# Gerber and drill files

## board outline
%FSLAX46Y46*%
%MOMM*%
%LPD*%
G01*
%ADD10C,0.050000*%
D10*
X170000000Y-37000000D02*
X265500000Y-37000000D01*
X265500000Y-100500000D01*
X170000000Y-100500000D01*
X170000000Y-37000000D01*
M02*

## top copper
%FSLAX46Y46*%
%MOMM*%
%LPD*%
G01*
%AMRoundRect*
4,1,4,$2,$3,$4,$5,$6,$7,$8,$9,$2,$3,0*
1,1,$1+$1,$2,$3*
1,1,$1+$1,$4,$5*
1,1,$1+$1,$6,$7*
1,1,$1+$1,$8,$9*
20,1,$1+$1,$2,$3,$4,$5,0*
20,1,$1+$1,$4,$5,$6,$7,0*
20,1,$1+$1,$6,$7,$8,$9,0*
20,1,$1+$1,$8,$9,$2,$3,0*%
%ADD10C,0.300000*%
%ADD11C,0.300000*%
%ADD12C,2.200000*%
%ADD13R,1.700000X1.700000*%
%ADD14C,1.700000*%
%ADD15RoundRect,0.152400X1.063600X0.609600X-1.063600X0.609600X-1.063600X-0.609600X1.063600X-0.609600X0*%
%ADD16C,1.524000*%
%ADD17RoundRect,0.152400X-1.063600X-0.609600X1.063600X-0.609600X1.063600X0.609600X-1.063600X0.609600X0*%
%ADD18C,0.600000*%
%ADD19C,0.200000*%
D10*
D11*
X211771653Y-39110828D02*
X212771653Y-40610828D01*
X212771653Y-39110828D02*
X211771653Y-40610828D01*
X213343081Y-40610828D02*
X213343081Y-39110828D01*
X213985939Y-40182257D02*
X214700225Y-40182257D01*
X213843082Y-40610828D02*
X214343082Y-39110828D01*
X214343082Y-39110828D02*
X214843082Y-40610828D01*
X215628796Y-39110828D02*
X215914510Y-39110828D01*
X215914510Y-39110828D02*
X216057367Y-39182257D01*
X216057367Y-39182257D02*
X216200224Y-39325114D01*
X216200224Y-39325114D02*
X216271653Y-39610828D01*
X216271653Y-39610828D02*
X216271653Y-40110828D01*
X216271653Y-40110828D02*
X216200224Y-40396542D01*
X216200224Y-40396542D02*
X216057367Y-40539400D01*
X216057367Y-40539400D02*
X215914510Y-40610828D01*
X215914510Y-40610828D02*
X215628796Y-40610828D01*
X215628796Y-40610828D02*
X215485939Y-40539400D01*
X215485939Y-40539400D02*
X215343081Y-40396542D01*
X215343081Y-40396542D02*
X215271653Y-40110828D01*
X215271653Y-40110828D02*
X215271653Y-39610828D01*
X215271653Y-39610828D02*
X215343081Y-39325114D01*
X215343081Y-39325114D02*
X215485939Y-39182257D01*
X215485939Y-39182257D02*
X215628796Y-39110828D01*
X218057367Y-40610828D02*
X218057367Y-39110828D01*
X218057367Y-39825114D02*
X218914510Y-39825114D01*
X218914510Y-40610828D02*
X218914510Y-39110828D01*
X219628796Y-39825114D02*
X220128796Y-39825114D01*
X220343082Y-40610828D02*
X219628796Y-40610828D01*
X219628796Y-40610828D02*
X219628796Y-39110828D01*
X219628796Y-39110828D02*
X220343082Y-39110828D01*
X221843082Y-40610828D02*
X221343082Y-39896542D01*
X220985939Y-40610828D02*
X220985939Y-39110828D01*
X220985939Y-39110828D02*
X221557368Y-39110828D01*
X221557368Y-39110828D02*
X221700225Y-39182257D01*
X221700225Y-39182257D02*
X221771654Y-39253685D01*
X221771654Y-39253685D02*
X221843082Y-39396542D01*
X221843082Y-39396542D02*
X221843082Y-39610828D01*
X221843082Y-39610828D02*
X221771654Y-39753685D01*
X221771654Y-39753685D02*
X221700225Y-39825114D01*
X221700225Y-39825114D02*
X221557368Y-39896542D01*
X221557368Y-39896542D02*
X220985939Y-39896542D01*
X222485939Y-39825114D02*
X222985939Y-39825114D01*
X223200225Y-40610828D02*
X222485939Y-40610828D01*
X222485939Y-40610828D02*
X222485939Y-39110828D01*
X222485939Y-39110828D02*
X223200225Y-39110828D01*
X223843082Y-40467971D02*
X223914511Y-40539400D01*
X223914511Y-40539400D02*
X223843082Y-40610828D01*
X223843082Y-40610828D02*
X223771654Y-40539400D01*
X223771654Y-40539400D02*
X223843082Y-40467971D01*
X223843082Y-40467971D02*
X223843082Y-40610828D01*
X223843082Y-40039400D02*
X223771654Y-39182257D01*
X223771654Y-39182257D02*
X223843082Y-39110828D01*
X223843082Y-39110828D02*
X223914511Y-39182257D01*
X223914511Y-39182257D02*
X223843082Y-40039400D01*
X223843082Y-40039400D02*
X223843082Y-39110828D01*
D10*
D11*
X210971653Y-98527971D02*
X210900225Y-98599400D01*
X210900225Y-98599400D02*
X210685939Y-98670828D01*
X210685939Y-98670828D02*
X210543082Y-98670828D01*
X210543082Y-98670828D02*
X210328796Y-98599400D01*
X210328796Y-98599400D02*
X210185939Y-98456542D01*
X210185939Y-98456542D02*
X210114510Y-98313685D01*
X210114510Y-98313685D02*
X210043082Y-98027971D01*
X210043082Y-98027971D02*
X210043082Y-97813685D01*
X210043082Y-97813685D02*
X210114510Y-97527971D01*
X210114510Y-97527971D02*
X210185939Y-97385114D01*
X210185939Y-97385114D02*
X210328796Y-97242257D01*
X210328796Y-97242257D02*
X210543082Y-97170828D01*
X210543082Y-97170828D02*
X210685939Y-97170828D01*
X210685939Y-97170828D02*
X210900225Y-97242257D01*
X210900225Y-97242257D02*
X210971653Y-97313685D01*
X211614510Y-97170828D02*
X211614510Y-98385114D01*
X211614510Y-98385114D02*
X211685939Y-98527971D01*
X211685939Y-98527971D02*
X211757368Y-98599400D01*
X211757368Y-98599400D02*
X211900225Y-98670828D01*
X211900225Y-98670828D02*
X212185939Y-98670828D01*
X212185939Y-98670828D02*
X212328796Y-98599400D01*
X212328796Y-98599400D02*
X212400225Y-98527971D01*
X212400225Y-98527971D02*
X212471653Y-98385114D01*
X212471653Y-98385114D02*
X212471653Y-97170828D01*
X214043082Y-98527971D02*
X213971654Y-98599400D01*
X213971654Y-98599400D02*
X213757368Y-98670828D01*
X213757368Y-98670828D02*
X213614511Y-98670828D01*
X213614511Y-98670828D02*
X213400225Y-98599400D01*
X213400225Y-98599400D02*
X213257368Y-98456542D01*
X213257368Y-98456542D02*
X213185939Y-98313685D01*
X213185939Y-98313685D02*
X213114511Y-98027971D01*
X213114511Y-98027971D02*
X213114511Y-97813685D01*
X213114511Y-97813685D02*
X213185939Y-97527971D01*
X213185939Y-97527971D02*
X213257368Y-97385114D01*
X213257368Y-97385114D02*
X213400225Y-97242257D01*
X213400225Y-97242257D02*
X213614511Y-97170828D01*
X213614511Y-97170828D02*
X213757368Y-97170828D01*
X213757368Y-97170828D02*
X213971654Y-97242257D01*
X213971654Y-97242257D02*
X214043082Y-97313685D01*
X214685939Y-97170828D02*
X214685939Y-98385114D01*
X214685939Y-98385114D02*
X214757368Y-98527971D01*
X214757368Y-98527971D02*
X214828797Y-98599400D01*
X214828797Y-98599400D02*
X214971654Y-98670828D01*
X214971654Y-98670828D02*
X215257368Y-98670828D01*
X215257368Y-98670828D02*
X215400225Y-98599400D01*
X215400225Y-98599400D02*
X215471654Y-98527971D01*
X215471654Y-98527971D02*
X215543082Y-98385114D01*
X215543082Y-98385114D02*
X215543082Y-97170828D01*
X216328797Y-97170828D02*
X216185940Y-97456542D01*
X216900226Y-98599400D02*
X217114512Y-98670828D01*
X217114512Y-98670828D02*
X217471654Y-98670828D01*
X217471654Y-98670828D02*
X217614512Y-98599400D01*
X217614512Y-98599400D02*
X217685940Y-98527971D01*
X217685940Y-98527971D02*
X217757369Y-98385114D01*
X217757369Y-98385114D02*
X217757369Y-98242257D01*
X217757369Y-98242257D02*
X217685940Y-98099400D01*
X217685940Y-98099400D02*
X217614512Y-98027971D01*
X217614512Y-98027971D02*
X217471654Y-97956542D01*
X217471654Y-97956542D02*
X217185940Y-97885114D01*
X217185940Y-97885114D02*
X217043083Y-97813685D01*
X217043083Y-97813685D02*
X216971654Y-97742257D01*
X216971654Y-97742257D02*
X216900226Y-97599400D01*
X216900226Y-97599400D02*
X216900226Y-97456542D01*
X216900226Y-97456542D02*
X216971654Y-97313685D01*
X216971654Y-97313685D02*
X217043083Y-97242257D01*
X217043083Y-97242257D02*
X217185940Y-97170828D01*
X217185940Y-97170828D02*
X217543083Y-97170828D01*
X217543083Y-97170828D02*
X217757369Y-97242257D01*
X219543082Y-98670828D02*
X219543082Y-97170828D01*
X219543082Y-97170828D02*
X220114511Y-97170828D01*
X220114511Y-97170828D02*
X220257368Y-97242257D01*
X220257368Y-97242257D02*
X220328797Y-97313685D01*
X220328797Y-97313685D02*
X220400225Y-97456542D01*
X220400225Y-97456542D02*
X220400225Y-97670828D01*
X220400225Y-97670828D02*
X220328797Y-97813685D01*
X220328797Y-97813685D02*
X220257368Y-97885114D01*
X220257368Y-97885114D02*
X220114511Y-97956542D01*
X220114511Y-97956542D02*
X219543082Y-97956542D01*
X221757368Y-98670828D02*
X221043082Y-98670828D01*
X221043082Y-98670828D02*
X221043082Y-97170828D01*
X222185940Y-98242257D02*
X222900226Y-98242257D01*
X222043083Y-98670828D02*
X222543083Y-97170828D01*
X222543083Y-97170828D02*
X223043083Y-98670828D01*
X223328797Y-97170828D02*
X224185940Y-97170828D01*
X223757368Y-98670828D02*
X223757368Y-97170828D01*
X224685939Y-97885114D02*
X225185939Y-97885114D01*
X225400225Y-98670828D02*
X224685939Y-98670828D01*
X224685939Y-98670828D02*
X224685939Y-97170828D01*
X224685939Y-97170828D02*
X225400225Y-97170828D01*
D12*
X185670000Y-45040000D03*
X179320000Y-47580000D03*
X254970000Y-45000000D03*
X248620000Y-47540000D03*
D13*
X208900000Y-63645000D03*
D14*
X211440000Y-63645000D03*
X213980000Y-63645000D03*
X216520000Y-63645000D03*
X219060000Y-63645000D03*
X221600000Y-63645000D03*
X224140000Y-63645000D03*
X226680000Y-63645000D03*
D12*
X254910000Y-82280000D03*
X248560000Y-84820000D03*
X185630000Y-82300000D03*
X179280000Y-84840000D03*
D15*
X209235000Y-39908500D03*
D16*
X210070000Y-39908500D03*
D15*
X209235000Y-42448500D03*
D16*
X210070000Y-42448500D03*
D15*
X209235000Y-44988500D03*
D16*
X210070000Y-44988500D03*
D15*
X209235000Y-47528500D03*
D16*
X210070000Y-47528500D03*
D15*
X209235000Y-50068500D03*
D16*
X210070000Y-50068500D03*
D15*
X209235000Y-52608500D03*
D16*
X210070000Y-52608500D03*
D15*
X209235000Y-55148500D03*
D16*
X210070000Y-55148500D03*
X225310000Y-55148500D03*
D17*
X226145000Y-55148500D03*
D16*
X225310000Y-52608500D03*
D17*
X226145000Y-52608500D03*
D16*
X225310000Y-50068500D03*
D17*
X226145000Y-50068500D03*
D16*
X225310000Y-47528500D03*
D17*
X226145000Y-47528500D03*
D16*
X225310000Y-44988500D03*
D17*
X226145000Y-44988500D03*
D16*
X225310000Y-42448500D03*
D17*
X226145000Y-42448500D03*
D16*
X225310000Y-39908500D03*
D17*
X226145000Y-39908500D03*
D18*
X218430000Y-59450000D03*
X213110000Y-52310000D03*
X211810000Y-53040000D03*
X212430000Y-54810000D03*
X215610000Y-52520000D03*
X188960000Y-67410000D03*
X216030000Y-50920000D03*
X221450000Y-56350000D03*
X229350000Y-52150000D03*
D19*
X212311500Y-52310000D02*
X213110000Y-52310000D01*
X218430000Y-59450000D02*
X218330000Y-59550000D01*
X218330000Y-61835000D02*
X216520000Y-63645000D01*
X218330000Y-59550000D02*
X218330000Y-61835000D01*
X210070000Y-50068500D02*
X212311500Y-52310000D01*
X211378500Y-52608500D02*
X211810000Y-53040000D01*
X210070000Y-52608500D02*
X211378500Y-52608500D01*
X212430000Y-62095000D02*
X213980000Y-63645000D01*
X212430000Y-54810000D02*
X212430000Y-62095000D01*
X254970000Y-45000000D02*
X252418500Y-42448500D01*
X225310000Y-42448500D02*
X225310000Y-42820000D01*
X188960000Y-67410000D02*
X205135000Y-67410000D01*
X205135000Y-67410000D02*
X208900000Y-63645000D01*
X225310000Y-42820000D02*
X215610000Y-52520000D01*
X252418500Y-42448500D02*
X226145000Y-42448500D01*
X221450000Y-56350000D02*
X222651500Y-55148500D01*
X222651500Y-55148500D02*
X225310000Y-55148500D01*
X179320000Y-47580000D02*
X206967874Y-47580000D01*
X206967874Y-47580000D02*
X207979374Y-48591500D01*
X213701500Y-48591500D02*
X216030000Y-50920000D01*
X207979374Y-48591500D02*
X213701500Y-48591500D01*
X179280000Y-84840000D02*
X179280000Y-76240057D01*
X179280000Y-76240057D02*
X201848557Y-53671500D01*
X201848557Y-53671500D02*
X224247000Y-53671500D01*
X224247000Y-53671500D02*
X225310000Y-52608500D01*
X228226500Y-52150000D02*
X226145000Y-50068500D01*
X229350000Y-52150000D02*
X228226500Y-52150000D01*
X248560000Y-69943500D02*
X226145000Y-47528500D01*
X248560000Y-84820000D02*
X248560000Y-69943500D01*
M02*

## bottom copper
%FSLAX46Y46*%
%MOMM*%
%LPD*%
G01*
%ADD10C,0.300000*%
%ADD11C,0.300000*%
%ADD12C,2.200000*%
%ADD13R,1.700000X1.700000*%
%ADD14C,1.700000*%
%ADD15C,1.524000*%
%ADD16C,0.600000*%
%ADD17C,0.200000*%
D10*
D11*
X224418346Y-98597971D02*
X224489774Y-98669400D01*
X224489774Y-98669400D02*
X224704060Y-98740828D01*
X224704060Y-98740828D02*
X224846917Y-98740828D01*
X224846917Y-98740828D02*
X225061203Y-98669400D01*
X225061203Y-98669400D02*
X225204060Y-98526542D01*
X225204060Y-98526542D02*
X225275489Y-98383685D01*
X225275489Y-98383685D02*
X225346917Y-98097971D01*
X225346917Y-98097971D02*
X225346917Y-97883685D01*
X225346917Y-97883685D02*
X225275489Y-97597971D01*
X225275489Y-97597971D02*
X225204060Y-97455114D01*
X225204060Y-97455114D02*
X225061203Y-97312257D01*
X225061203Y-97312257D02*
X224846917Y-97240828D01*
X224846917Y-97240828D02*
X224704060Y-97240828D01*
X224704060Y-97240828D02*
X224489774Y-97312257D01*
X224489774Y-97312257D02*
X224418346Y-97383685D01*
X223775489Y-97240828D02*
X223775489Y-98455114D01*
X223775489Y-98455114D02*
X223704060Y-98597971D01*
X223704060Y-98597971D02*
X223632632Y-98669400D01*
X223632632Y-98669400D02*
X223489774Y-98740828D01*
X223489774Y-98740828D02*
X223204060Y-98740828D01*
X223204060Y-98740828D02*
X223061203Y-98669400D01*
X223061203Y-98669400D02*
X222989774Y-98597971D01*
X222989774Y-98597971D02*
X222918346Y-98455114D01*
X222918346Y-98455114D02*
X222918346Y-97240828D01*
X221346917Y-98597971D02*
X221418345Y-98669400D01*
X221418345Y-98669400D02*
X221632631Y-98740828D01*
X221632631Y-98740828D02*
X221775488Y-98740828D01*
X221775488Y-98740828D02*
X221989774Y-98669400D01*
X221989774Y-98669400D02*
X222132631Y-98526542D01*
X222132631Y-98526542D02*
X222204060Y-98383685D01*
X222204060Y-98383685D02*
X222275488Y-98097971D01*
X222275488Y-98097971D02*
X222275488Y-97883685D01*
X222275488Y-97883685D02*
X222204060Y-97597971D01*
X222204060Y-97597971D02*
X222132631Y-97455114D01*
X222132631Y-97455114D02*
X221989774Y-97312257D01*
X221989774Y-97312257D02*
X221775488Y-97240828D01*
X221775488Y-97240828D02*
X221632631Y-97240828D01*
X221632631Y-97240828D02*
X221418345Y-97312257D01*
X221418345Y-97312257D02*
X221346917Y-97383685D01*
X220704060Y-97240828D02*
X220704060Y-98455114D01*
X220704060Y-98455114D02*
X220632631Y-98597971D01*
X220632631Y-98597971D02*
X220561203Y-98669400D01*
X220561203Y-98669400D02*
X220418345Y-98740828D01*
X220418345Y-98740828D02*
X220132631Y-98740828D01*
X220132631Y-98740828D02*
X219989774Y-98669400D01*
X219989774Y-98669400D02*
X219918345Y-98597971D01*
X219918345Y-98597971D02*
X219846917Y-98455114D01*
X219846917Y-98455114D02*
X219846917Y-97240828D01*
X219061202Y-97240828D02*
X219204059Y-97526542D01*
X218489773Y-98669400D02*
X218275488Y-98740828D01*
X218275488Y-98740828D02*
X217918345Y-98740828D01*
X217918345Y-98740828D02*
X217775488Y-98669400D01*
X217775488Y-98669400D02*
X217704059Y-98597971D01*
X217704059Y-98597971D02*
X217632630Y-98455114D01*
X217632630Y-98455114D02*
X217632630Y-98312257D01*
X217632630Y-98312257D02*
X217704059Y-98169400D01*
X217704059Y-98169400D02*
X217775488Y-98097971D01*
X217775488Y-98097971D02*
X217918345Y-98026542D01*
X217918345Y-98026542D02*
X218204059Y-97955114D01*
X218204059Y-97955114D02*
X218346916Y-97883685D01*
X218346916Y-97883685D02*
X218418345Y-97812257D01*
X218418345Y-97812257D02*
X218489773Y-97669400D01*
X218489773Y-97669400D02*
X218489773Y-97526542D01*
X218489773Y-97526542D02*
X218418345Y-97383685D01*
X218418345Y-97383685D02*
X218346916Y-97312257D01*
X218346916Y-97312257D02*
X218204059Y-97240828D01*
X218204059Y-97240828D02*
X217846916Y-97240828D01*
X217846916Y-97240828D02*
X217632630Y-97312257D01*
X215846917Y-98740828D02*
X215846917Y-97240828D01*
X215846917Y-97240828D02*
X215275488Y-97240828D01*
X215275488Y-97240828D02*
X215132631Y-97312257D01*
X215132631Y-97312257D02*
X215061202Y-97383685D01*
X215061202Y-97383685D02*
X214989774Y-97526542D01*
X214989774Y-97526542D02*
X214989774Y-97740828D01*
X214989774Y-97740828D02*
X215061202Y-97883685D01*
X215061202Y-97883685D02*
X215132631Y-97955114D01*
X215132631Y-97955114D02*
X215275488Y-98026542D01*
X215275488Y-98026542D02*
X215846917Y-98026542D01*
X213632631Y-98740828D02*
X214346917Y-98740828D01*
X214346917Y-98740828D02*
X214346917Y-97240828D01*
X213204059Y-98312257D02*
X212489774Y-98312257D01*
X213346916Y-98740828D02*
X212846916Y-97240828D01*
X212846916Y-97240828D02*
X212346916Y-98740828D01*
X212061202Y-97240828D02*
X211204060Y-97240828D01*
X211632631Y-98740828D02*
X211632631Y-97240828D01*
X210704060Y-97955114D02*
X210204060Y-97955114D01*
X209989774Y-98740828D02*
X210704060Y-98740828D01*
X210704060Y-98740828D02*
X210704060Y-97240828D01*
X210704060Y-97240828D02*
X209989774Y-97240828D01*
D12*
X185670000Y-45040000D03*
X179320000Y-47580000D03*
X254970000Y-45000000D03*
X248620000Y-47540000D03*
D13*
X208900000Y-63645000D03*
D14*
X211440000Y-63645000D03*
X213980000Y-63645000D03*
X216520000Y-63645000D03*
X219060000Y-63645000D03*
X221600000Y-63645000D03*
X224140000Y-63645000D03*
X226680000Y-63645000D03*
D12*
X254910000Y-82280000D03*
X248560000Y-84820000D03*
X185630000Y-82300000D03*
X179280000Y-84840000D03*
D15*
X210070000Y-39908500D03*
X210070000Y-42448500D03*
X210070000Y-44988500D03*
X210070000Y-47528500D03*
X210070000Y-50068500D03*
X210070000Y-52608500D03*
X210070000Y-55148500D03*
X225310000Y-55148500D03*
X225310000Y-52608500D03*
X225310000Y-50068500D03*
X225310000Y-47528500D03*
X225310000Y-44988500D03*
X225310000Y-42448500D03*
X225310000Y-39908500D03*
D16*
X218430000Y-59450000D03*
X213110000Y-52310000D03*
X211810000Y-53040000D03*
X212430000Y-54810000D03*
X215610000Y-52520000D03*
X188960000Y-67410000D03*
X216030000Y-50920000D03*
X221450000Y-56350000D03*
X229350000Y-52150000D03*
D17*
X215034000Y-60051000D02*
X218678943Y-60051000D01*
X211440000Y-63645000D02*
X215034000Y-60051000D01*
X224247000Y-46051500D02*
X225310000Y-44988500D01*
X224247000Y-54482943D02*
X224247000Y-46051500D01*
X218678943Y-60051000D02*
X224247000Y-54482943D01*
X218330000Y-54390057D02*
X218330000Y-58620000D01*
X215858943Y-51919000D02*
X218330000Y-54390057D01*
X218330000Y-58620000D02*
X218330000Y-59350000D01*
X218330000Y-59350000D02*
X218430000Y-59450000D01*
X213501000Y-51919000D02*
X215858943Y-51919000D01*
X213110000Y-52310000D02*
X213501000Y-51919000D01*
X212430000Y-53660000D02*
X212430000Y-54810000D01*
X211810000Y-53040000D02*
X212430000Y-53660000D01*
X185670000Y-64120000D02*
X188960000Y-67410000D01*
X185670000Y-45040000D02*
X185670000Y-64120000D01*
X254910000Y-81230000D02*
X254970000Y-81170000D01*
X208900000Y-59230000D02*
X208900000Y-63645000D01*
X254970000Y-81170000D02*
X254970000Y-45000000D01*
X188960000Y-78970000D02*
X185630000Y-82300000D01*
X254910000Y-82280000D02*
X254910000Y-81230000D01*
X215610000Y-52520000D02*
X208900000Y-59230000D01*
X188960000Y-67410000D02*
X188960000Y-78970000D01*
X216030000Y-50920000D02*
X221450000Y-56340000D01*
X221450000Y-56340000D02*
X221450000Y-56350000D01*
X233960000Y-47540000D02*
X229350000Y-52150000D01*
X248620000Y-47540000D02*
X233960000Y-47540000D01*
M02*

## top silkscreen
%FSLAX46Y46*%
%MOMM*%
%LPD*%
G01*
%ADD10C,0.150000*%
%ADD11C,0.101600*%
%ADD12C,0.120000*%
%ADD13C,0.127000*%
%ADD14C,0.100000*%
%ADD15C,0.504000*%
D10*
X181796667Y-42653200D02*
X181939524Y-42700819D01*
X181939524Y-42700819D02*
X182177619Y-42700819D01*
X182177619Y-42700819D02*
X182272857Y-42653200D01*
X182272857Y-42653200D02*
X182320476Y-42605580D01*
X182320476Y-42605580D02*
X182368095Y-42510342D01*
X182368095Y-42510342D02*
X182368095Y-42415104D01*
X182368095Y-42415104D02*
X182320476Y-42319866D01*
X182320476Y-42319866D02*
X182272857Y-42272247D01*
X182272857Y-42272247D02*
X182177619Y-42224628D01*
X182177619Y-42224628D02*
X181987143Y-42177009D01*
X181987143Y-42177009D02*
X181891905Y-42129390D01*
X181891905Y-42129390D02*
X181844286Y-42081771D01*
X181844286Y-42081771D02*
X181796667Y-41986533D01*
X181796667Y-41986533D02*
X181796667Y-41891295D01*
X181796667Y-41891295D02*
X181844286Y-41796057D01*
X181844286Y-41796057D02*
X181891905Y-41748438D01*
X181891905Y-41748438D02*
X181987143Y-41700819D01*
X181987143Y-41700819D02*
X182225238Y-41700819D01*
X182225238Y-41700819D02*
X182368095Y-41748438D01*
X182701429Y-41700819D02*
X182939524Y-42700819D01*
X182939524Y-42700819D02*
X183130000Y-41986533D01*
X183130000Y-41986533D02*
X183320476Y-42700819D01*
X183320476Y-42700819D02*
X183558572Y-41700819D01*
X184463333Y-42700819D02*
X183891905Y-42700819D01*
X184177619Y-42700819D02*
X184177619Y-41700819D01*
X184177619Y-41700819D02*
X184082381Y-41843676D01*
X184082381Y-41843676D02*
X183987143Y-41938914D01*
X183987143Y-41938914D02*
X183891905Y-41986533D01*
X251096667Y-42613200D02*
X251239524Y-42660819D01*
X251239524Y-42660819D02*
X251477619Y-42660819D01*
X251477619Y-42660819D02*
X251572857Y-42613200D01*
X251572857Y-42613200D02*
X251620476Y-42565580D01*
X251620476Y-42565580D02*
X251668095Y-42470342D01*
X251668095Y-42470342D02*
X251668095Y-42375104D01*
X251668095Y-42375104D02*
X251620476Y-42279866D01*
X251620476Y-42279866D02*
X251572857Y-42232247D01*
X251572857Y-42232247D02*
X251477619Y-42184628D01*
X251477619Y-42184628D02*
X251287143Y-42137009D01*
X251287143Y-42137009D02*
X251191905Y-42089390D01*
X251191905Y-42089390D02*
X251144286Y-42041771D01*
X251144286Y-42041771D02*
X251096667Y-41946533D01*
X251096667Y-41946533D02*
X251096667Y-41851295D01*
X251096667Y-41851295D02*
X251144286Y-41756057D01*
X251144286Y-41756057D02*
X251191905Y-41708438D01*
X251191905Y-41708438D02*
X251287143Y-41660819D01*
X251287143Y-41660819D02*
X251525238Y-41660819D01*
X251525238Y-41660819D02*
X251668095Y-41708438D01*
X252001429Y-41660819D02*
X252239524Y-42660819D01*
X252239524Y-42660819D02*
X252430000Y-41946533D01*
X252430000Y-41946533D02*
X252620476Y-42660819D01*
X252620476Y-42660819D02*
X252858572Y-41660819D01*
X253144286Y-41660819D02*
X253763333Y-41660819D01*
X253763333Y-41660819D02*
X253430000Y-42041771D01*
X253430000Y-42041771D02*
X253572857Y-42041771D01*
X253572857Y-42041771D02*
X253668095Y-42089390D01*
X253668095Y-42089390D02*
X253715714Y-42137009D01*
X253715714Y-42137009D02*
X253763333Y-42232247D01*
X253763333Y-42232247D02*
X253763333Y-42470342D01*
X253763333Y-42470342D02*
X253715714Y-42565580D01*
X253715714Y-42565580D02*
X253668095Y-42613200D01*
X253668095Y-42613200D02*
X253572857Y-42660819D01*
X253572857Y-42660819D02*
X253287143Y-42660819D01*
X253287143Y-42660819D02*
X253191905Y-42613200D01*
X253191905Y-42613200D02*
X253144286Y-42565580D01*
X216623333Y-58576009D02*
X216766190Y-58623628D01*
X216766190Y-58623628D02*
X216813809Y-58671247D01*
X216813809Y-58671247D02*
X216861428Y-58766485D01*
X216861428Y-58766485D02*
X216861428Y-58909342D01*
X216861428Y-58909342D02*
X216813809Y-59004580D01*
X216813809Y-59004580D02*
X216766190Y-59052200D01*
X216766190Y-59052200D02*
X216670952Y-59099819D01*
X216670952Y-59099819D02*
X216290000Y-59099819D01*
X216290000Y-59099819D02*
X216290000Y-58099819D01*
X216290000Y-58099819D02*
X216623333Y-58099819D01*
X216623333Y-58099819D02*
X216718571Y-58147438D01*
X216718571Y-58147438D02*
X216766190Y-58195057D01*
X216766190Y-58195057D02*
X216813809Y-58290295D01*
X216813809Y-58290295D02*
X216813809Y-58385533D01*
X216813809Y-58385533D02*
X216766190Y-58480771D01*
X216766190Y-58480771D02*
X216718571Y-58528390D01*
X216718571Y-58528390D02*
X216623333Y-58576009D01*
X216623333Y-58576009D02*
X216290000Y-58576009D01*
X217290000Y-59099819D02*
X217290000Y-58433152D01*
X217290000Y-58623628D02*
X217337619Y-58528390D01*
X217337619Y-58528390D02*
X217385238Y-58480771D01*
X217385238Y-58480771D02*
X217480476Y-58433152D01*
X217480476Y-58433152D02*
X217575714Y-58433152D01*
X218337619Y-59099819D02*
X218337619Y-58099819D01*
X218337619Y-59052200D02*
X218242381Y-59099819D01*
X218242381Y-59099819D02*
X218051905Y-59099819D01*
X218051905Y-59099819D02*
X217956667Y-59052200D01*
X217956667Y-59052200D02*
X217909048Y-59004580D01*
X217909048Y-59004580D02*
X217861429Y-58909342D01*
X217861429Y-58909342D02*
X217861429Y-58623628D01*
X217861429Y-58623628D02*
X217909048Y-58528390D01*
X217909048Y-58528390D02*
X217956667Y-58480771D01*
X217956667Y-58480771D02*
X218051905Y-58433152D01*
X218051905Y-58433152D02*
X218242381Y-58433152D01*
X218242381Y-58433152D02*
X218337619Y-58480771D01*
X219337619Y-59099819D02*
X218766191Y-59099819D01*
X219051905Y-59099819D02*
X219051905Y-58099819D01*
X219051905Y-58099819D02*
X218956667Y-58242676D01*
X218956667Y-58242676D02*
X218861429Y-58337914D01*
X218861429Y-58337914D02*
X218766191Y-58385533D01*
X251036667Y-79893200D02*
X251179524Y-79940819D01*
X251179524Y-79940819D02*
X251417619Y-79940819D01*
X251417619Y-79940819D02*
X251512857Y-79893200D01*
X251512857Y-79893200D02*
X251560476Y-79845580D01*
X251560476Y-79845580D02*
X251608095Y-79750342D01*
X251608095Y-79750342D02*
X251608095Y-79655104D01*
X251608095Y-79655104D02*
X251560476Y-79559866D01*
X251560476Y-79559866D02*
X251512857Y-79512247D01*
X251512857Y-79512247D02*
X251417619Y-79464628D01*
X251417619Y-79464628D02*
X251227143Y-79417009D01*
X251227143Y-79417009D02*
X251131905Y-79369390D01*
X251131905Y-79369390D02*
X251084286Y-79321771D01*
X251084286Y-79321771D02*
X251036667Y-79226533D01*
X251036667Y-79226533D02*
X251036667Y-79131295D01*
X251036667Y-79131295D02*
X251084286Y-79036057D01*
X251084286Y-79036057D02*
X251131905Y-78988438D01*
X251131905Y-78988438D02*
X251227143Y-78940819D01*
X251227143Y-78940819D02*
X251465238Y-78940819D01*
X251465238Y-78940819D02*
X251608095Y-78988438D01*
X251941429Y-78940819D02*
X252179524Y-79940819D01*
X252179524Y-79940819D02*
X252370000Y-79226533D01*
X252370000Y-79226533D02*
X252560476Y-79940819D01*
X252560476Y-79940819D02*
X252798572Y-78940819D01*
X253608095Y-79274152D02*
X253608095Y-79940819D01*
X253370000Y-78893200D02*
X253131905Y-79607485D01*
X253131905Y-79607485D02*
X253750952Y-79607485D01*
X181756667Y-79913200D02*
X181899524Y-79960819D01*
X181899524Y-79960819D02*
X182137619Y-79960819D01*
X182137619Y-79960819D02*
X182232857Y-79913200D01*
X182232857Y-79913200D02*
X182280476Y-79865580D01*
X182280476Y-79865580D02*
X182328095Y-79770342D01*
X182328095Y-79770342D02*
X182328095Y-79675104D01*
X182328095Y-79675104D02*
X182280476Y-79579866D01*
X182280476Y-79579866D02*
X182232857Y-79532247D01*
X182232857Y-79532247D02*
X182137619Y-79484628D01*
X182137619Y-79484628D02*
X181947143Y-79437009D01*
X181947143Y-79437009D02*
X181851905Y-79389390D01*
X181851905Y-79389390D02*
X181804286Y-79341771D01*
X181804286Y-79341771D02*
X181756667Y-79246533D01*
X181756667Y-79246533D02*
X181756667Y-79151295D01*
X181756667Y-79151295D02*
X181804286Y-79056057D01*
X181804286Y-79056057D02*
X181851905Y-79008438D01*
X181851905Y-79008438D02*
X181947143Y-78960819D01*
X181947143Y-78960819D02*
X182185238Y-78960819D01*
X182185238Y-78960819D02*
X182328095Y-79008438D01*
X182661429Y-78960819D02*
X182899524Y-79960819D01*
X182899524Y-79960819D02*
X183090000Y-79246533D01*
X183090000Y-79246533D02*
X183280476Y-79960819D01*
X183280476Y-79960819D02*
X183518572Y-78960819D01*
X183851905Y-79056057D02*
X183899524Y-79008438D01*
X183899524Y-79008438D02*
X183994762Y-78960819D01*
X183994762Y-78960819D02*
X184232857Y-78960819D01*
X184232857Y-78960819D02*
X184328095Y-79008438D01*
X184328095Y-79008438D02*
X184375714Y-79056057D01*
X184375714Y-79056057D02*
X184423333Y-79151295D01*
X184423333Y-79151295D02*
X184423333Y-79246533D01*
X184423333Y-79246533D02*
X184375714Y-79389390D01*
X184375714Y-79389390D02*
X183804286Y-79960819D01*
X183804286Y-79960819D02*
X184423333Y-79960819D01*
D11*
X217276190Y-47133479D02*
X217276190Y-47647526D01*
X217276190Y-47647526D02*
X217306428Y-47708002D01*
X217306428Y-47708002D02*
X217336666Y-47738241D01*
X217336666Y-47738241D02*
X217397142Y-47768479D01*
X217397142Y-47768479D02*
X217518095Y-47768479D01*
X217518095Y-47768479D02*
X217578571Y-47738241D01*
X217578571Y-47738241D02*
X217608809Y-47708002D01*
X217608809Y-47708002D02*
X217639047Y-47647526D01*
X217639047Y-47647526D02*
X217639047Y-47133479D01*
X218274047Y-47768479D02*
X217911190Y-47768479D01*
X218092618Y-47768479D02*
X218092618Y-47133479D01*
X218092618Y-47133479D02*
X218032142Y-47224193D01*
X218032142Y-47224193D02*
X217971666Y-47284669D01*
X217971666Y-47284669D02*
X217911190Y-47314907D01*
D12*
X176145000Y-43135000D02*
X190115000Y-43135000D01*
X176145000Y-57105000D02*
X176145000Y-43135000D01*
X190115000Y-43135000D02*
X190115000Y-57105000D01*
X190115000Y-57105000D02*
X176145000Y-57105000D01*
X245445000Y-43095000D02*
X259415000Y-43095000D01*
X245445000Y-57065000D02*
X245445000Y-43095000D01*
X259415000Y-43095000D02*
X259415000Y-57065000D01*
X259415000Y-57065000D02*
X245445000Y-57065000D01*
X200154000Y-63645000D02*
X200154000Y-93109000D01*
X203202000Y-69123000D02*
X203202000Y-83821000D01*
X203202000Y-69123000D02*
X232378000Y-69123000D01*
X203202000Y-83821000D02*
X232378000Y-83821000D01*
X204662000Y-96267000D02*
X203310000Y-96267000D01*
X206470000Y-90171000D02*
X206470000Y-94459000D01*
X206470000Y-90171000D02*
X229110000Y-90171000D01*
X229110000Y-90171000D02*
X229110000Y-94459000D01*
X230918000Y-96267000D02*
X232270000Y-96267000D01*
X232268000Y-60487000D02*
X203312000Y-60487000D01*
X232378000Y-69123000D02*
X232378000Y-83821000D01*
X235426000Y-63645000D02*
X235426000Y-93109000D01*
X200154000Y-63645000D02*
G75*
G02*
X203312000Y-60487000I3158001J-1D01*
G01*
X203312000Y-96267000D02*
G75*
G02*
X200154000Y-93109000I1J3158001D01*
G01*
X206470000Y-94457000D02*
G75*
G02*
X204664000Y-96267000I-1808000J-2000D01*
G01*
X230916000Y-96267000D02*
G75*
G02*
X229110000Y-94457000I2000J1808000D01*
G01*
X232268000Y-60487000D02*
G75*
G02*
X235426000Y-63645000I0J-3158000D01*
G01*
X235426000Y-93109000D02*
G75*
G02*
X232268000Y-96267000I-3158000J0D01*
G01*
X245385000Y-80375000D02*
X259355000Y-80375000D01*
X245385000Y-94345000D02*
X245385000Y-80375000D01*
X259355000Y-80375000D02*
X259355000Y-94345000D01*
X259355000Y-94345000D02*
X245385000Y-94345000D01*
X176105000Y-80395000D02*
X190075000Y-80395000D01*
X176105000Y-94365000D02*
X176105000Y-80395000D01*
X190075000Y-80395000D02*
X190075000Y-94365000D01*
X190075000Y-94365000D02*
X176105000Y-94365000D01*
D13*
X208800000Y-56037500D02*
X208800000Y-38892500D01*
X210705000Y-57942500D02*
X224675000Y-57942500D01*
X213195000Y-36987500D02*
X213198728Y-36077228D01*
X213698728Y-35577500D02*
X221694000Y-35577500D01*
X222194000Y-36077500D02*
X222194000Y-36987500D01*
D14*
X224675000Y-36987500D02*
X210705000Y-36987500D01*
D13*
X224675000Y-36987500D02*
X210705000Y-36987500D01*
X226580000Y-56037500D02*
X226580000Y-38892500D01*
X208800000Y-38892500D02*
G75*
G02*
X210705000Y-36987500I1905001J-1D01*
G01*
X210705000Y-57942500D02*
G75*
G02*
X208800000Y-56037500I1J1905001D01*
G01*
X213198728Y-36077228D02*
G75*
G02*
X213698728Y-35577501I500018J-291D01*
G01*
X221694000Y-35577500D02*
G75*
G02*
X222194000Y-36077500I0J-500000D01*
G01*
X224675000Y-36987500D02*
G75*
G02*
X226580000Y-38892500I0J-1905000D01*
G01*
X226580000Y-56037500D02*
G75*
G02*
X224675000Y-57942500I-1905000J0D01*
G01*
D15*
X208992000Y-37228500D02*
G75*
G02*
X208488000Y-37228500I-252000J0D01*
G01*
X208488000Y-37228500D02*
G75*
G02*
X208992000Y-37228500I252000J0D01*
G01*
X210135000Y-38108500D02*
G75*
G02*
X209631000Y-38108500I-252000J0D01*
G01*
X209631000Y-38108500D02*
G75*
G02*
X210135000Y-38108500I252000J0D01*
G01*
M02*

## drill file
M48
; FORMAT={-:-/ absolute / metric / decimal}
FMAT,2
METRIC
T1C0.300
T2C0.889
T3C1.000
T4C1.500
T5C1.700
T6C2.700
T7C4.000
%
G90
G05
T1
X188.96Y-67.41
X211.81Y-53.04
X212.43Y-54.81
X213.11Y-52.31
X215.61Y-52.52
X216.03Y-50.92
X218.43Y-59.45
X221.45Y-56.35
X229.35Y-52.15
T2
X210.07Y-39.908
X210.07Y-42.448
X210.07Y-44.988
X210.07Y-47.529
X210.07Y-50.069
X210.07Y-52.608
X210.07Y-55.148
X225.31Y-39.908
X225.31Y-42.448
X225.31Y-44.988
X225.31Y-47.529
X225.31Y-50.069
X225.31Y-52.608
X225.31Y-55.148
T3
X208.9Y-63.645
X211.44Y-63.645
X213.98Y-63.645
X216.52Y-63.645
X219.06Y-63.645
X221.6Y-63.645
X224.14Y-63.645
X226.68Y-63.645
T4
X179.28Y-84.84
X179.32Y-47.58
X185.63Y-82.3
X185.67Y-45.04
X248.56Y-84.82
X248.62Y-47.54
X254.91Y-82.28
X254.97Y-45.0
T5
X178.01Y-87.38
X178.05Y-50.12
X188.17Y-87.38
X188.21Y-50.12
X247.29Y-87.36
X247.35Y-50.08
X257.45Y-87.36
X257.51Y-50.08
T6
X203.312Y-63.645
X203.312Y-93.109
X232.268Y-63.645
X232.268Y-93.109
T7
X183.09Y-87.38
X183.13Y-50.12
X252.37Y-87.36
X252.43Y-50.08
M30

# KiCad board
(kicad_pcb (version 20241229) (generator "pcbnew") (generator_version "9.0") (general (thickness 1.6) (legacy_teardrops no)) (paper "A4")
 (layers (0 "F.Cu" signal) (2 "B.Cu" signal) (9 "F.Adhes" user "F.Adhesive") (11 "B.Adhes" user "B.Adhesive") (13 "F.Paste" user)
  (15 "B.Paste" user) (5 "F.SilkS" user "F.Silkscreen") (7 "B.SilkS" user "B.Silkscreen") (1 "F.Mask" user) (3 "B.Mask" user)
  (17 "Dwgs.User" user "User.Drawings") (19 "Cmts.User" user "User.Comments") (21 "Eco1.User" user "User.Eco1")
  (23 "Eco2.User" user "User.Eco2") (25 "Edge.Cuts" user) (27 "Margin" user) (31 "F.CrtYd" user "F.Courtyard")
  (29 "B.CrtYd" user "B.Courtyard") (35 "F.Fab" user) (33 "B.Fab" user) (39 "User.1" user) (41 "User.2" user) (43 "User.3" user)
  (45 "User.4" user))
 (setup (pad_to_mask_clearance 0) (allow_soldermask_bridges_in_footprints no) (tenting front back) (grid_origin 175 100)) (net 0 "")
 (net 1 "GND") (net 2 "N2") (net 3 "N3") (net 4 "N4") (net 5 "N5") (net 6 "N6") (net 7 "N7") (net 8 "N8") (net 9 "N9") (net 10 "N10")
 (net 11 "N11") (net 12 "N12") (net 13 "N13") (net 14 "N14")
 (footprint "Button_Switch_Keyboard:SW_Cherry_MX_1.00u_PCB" (layer "F.Cu") (at 185.67 45.04)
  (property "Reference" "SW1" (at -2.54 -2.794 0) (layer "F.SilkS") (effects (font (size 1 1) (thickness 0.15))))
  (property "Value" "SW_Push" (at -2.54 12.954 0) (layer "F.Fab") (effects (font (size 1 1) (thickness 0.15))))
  (fp_line (start -9.525 -1.905) (end 4.445 -1.905) (stroke (width 0.12) (type solid)) (layer "F.SilkS"))
  (fp_line (start -9.525 12.065) (end -9.525 -1.905) (stroke (width 0.12) (type solid)) (layer "F.SilkS"))
  (fp_line (start 4.445 -1.905) (end 4.445 12.065) (stroke (width 0.12) (type solid)) (layer "F.SilkS"))
  (fp_line (start 4.445 12.065) (end -9.525 12.065) (stroke (width 0.12) (type solid)) (layer "F.SilkS"))
  (pad "" np_thru_hole circle (at -7.62 5.08) (size 1.7 1.7) (drill 1.7) (layers "*.Cu" "*.Mask"))
  (pad "" np_thru_hole circle (at -2.54 5.08) (size 4 4) (drill 4) (layers "*.Cu" "*.Mask"))
  (pad "" np_thru_hole circle (at 2.54 5.08) (size 1.7 1.7) (drill 1.7) (layers "*.Cu" "*.Mask"))
  (pad "1" thru_hole circle (at 0 0) (size 2.2 2.2) (drill 1.5) (layers "*.Cu" "*.Mask") (remove_unused_layers no) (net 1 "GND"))
  (pad "2" thru_hole circle (at -6.35 2.54) (size 2.2 2.2) (drill 1.5) (layers "*.Cu" "*.Mask") (remove_unused_layers no) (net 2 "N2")))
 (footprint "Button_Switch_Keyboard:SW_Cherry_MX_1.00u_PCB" (layer "F.Cu") (at 254.97 45)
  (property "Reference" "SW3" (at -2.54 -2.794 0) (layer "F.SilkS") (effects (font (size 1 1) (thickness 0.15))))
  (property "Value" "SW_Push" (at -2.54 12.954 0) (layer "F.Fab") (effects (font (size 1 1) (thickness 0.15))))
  (fp_line (start -9.525 -1.905) (end 4.445 -1.905) (stroke (width 0.12) (type solid)) (layer "F.SilkS"))
  (fp_line (start -9.525 12.065) (end -9.525 -1.905) (stroke (width 0.12) (type solid)) (layer "F.SilkS"))
  (fp_line (start 4.445 -1.905) (end 4.445 12.065) (stroke (width 0.12) (type solid)) (layer "F.SilkS"))
  (fp_line (start 4.445 12.065) (end -9.525 12.065) (stroke (width 0.12) (type solid)) (layer "F.SilkS"))
  (pad "" np_thru_hole circle (at -7.62 5.08) (size 1.7 1.7) (drill 1.7) (layers "*.Cu" "*.Mask"))
  (pad "" np_thru_hole circle (at -2.54 5.08) (size 4 4) (drill 4) (layers "*.Cu" "*.Mask"))
  (pad "" np_thru_hole circle (at 2.54 5.08) (size 1.7 1.7) (drill 1.7) (layers "*.Cu" "*.Mask"))
  (pad "1" thru_hole circle (at 0 0) (size 2.2 2.2) (drill 1.5) (layers "*.Cu" "*.Mask") (remove_unused_layers no) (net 1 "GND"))
  (pad "2" thru_hole circle (at -6.35 2.54) (size 2.2 2.2) (drill 1.5) (layers "*.Cu" "*.Mask") (remove_unused_layers no) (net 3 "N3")))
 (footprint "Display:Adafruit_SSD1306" (layer "F.Cu") (at 208.9 63.645)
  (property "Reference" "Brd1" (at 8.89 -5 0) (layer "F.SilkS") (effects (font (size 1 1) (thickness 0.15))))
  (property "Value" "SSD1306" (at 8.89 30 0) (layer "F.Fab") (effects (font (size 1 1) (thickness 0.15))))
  (fp_line (start -8.746 0) (end -8.746 29.464) (stroke (width 0.12) (type solid)) (layer "F.SilkS"))
  (fp_line (start -5.698 5.478) (end -5.698 20.176) (stroke (width 0.12) (type solid)) (layer "F.SilkS"))
  (fp_line (start -5.698 5.478) (end 23.478 5.478) (stroke (width 0.12) (type solid)) (layer "F.SilkS"))
  (fp_line (start -5.698 20.176) (end 23.478 20.176) (stroke (width 0.12) (type solid)) (layer "F.SilkS"))
  (fp_line (start -4.238 32.622) (end -5.59 32.622) (stroke (width 0.12) (type solid)) (layer "F.SilkS"))
  (fp_line (start -2.43 26.526) (end -2.43 30.814) (stroke (width 0.12) (type solid)) (layer "F.SilkS"))
  (fp_line (start -2.43 26.526) (end 20.21 26.526) (stroke (width 0.12) (type solid)) (layer "F.SilkS"))
  (fp_line (start 20.21 26.526) (end 20.21 30.814) (stroke (width 0.12) (type solid)) (layer "F.SilkS"))
  (fp_line (start 22.018 32.622) (end 23.37 32.622) (stroke (width 0.12) (type solid)) (layer "F.SilkS"))
  (fp_line (start 23.368 -3.158) (end -5.588 -3.158) (stroke (width 0.12) (type solid)) (layer "F.SilkS"))
  (fp_line (start 23.478 5.478) (end 23.478 20.176) (stroke (width 0.12) (type solid)) (layer "F.SilkS"))
  (fp_line (start 26.526 0) (end 26.526 29.464) (stroke (width 0.12) (type solid)) (layer "F.SilkS"))
  (fp_arc (start -8.746 0) (mid -7.821043 -2.233043) (end -5.588 -3.158) (stroke (width 0.12) (type solid)) (layer "F.SilkS"))
  (fp_arc (start -5.588 32.622) (mid -7.821043 31.697043) (end -8.746 29.464) (stroke (width 0.12) (type solid)) (layer "F.SilkS"))
  (fp_arc (start -2.43 30.812) (mid -2.958137 32.091035) (end -4.236 32.622) (stroke (width 0.12) (type solid)) (layer "F.SilkS"))
  (fp_arc (start 22.016 32.622) (mid 20.738137 32.091035) (end 20.21 30.812) (stroke (width 0.12) (type solid)) (layer "F.SilkS"))
  (fp_arc (start 23.368 -3.158) (mid 25.601043 -2.233043) (end 26.526 0) (stroke (width 0.12) (type solid)) (layer "F.SilkS"))
  (fp_arc (start 26.526 29.464) (mid 25.601043 31.697043) (end 23.368 32.622) (stroke (width 0.12) (type solid)) (layer "F.SilkS"))
  (pad "" np_thru_hole circle (at -5.588 0) (size 2.7 2.7) (drill 2.7) (layers "*.Cu" "*.Mask"))
  (pad "" np_thru_hole circle (at -5.588 29.464) (size 2.7 2.7) (drill 2.7) (layers "*.Cu" "*.Mask"))
  (pad "" np_thru_hole circle (at 23.368 0) (size 2.7 2.7) (drill 2.7) (layers "*.Cu" "*.Mask"))
  (pad "" np_thru_hole circle (at 23.368 29.464) (size 2.7 2.7) (drill 2.7) (layers "*.Cu" "*.Mask"))
  (pad "1" thru_hole rect (at 0 0) (size 1.7 1.7) (drill 1) (layers "*.Cu" "*.Mask") (remove_unused_layers no) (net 1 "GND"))
  (pad "2" thru_hole circle (at 2.54 0) (size 1.7 1.7) (drill 1) (layers "*.Cu" "*.Mask") (remove_unused_layers no) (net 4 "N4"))
  (pad "3" thru_hole circle (at 5.08 0) (size 1.7 1.7) (drill 1) (layers "*.Cu" "*.Mask") (remove_unused_layers no) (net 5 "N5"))
  (pad "4" thru_hole circle (at 7.62 0) (size 1.7 1.7) (drill 1) (layers "*.Cu" "*.Mask") (remove_unused_layers no) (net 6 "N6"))
  (pad "5" thru_hole circle (at 10.16 0) (size 1.7 1.7) (drill 1) (layers "*.Cu" "*.Mask") (remove_unused_layers no))
  (pad "6" thru_hole circle (at 12.7 0) (size 1.7 1.7) (drill 1) (layers "*.Cu" "*.Mask") (remove_unused_layers no))
  (pad "7" thru_hole circle (at 15.24 0) (size 1.7 1.7) (drill 1) (layers "*.Cu" "*.Mask") (remove_unused_layers no))
  (pad "8" thru_hole circle (at 17.78 0) (size 1.7 1.7) (drill 1) (layers "*.Cu" "*.Mask") (remove_unused_layers no)))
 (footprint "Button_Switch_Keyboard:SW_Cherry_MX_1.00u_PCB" (layer "F.Cu") (at 254.91 82.28)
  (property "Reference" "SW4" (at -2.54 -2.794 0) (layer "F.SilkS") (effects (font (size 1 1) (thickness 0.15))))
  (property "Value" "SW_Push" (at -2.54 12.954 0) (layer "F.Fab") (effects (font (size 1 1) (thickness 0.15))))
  (fp_line (start -9.525 -1.905) (end 4.445 -1.905) (stroke (width 0.12) (type solid)) (layer "F.SilkS"))
  (fp_line (start -9.525 12.065) (end -9.525 -1.905) (stroke (width 0.12) (type solid)) (layer "F.SilkS"))
  (fp_line (start 4.445 -1.905) (end 4.445 12.065) (stroke (width 0.12) (type solid)) (layer "F.SilkS"))
  (fp_line (start 4.445 12.065) (end -9.525 12.065) (stroke (width 0.12) (type solid)) (layer "F.SilkS"))
  (pad "" np_thru_hole circle (at -7.62 5.08) (size 1.7 1.7) (drill 1.7) (layers "*.Cu" "*.Mask"))
  (pad "" np_thru_hole circle (at -2.54 5.08) (size 4 4) (drill 4) (layers "*.Cu" "*.Mask"))
  (pad "" np_thru_hole circle (at 2.54 5.08) (size 1.7 1.7) (drill 1.7) (layers "*.Cu" "*.Mask"))
  (pad "1" thru_hole circle (at 0 0) (size 2.2 2.2) (drill 1.5) (layers "*.Cu" "*.Mask") (remove_unused_layers no) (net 1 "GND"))
  (pad "2" thru_hole circle (at -6.35 2.54) (size 2.2 2.2) (drill 1.5) (layers "*.Cu" "*.Mask") (remove_unused_layers no) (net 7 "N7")))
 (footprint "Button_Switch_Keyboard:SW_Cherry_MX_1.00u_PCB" (layer "F.Cu") (at 185.63 82.3)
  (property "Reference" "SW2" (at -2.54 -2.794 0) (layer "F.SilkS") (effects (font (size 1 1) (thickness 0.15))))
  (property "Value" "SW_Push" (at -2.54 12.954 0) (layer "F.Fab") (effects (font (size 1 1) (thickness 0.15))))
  (fp_line (start -9.525 -1.905) (end 4.445 -1.905) (stroke (width 0.12) (type solid)) (layer "F.SilkS"))
  (fp_line (start -9.525 12.065) (end -9.525 -1.905) (stroke (width 0.12) (type solid)) (layer "F.SilkS"))
  (fp_line (start 4.445 -1.905) (end 4.445 12.065) (stroke (width 0.12) (type solid)) (layer "F.SilkS"))
  (fp_line (start 4.445 12.065) (end -9.525 12.065) (stroke (width 0.12) (type solid)) (layer "F.SilkS"))
  (pad "" np_thru_hole circle (at -7.62 5.08) (size 1.7 1.7) (drill 1.7) (layers "*.Cu" "*.Mask"))
  (pad "" np_thru_hole circle (at -2.54 5.08) (size 4 4) (drill 4) (layers "*.Cu" "*.Mask"))
  (pad "" np_thru_hole circle (at 2.54 5.08) (size 1.7 1.7) (drill 1.7) (layers "*.Cu" "*.Mask"))
  (pad "1" thru_hole circle (at 0 0) (size 2.2 2.2) (drill 1.5) (layers "*.Cu" "*.Mask") (remove_unused_layers no) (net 1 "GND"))
  (pad "2" thru_hole circle (at -6.35 2.54) (size 2.2 2.2) (drill 1.5) (layers "*.Cu" "*.Mask") (remove_unused_layers no) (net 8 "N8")))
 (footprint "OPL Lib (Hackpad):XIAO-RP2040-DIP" (layer "F.Cu") (at 217.69 47.5285)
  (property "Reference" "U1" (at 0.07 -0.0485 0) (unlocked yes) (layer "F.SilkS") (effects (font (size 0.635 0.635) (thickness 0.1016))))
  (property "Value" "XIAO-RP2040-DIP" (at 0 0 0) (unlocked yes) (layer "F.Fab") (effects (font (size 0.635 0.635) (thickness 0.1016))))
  (fp_line (start -8.89 8.509) (end -8.89 -8.636) (stroke (width 0.127) (type solid)) (layer "F.SilkS"))
  (fp_line (start -6.985 10.414) (end 6.985 10.414) (stroke (width 0.127) (type solid)) (layer "F.SilkS"))
  (fp_line (start -4.495 -10.541) (end -4.491272 -11.451272) (stroke (width 0.127) (type solid)) (layer "F.SilkS"))
  (fp_line (start -3.991272 -11.951) (end 4.004 -11.951) (stroke (width 0.127) (type solid)) (layer "F.SilkS"))
  (fp_line (start 4.504 -11.451) (end 4.504 -10.541) (stroke (width 0.127) (type solid)) (layer "F.SilkS"))
  (fp_line (start 6.985 -10.541) (end -6.985 -10.541) (stroke (width 0.1) (type solid)) (layer "F.SilkS"))
  (fp_line (start 6.985 -10.541) (end -6.985 -10.541) (stroke (width 0.127) (type solid)) (layer "F.SilkS"))
  (fp_line (start 8.89 8.509) (end 8.89 -8.636) (stroke (width 0.127) (type solid)) (layer "F.SilkS"))
  (fp_arc (start -8.89 -8.636) (mid -8.332038 -9.983038) (end -6.985 -10.541) (stroke (width 0.127) (type solid)) (layer "F.SilkS"))
  (fp_arc (start -6.985 10.414) (mid -8.332038 9.856038) (end -8.89 8.509) (stroke (width 0.127) (type solid)) (layer "F.SilkS"))
  (fp_arc (start -4.491272 -11.451272) (mid -4.344728 -11.80464) (end -3.991272 -11.951) (stroke (width 0.127) (type default))
   (layer "F.SilkS"))
  (fp_arc (start 4.004 -11.951) (mid 4.357553 -11.804553) (end 4.504 -11.451) (stroke (width 0.127) (type default)) (layer "F.SilkS"))
  (fp_arc (start 6.985 -10.541) (mid 8.332038 -9.983038) (end 8.89 -8.636) (stroke (width 0.127) (type solid)) (layer "F.SilkS"))
  (fp_arc (start 8.89 8.509) (mid 8.332038 9.856038) (end 6.985 10.414) (stroke (width 0.127) (type solid)) (layer "F.SilkS"))
  (fp_circle (center -8.95 -10.3) (end -8.95 -10.554) (stroke (width 0.5) (type solid)) (fill yes) (layer "F.SilkS"))
  (fp_circle (center -7.807 -9.42) (end -7.807 -9.674) (stroke (width 0.5) (type solid)) (fill yes) (layer "F.SilkS"))
  (pad "1" smd roundrect (at -8.455 -7.62 180) (size 2.432 1.524) (layers "F.Cu" "F.Mask") (roundrect_rratio 0.1) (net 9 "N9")
   (thermal_bridge_angle 45))
  (pad "1" thru_hole circle (at -7.62 -7.62 180) (size 1.524 1.524) (drill 0.889) (layers "*.Cu" "*.Mask") (remove_unused_layers no)
   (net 9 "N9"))
  (pad "2" smd roundrect (at -8.455 -5.08 180) (size 2.432 1.524) (layers "F.Cu" "F.Mask") (roundrect_rratio 0.1) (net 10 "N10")
   (thermal_bridge_angle 45))
  (pad "2" thru_hole circle (at -7.62 -5.08 180) (size 1.524 1.524) (drill 0.889) (layers "*.Cu" "*.Mask") (remove_unused_layers no)
   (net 10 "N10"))
  (pad "3" smd roundrect (at -8.455 -2.54 180) (size 2.432 1.524) (layers "F.Cu" "F.Mask") (roundrect_rratio 0.1) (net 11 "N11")
   (thermal_bridge_angle 45))
  (pad "3" thru_hole circle (at -7.62 -2.54 180) (size 1.524 1.524) (drill 0.889) (layers "*.Cu" "*.Mask") (remove_unused_layers no)
   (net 11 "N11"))
  (pad "4" smd roundrect (at -8.455 0 180) (size 2.432 1.524) (layers "F.Cu" "F.Mask") (roundrect_rratio 0.1) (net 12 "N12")
   (thermal_bridge_angle 45))
  (pad "4" thru_hole circle (at -7.62 0 180) (size 1.524 1.524) (drill 0.889) (layers "*.Cu" "*.Mask") (remove_unused_layers no)
   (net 12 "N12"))
  (pad "5" smd roundrect (at -8.455 2.54 180) (size 2.432 1.524) (layers "F.Cu" "F.Mask") (roundrect_rratio 0.1) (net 6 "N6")
   (thermal_bridge_angle 45))
  (pad "5" thru_hole circle (at -7.62 2.54 180) (size 1.524 1.524) (drill 0.889) (layers "*.Cu" "*.Mask") (remove_unused_layers no)
   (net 6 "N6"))
  (pad "6" smd roundrect (at -8.455 5.08 180) (size 2.432 1.524) (layers "F.Cu" "F.Mask") (roundrect_rratio 0.1) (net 5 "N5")
   (thermal_bridge_angle 45))
  (pad "6" thru_hole circle (at -7.62 5.08 180) (size 1.524 1.524) (drill 0.889) (layers "*.Cu" "*.Mask") (remove_unused_layers no)
   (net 5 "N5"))
  (pad "7" smd roundrect (at -8.455 7.62 180) (size 2.432 1.524) (layers "F.Cu" "F.Mask") (roundrect_rratio 0.1) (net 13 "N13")
   (thermal_bridge_angle 45))
  (pad "7" thru_hole circle (at -7.62 7.62 180) (size 1.524 1.524) (drill 0.889) (layers "*.Cu" "*.Mask") (remove_unused_layers no)
   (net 13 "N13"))
  (pad "8" thru_hole circle (at 7.62 7.62) (size 1.524 1.524) (drill 0.889) (layers "*.Cu" "*.Mask") (remove_unused_layers no) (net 2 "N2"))
  (pad "8" smd roundrect (at 8.455 7.62) (size 2.432 1.524) (layers "F.Cu" "F.Mask") (roundrect_rratio 0.1) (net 2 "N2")
   (thermal_bridge_angle 45))
  (pad "9" thru_hole circle (at 7.62 5.08) (size 1.524 1.524) (drill 0.889) (layers "*.Cu" "*.Mask") (remove_unused_layers no) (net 8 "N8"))
  (pad "9" smd roundrect (at 8.455 5.08) (size 2.432 1.524) (layers "F.Cu" "F.Mask") (roundrect_rratio 0.1) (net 8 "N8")
   (thermal_bridge_angle 45))
  (pad "10" thru_hole circle (at 7.62 2.54) (size 1.524 1.524) (drill 0.889) (layers "*.Cu" "*.Mask") (remove_unused_layers no) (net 3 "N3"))
  (pad "10" smd roundrect (at 8.455 2.54) (size 2.432 1.524) (layers "F.Cu" "F.Mask") (roundrect_rratio 0.1) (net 3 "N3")
   (thermal_bridge_angle 45))
  (pad "11" thru_hole circle (at 7.62 0) (size 1.524 1.524) (drill 0.889) (layers "*.Cu" "*.Mask") (remove_unused_layers no) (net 7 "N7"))
  (pad "11" smd roundrect (at 8.455 0) (size 2.432 1.524) (layers "F.Cu" "F.Mask") (roundrect_rratio 0.1) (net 7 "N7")
   (thermal_bridge_angle 45))
  (pad "12" thru_hole circle (at 7.62 -2.54) (size 1.524 1.524) (drill 0.889) (layers "*.Cu" "*.Mask") (remove_unused_layers no)
   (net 4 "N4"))
  (pad "12" smd roundrect (at 8.455 -2.54) (size 2.432 1.524) (layers "F.Cu" "F.Mask") (roundrect_rratio 0.1) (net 4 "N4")
   (thermal_bridge_angle 45))
  (pad "13" thru_hole circle (at 7.62 -5.08) (size 1.524 1.524) (drill 0.889) (layers "*.Cu" "*.Mask") (remove_unused_layers no)
   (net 1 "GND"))
  (pad "13" smd roundrect (at 8.455 -5.08) (size 2.432 1.524) (layers "F.Cu" "F.Mask") (roundrect_rratio 0.1) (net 1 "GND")
   (thermal_bridge_angle 45))
  (pad "14" thru_hole circle (at 7.62 -7.62) (size 1.524 1.524) (drill 0.889) (layers "*.Cu" "*.Mask") (remove_unused_layers no)
   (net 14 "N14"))
  (pad "14" smd roundrect (at 8.455 -7.62) (size 2.432 1.524) (layers "F.Cu" "F.Mask") (roundrect_rratio 0.1) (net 14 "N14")
   (thermal_bridge_angle 45)))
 (gr_rect (start 170 37) (end 265.5 100.5) (stroke (width 0.05) (type default)) (fill no) (layer "Edge.Cuts"))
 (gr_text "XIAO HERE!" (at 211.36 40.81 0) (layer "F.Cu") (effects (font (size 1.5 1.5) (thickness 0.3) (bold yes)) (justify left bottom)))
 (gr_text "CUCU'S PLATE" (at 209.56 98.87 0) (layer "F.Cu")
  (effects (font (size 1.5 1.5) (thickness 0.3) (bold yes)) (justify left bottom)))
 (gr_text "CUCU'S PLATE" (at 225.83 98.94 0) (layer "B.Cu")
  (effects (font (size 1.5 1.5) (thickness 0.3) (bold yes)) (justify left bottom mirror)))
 (segment (start 215.034 60.051) (end 218.678943 60.051) (width 0.2) (layer "B.Cu") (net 4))
 (segment (start 211.44 63.645) (end 215.034 60.051) (width 0.2) (layer "B.Cu") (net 4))
 (segment (start 224.247 46.0515) (end 225.31 44.9885) (width 0.2) (layer "B.Cu") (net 4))
 (segment (start 224.247 54.482943) (end 224.247 46.0515) (width 0.2) (layer "B.Cu") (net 4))
 (segment (start 218.678943 60.051) (end 224.247 54.482943) (width 0.2) (layer "B.Cu") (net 4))
 (segment (start 212.3115 52.31) (end 213.11 52.31) (width 0.2) (layer "F.Cu") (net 6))
 (segment (start 218.43 59.45) (end 218.33 59.55) (width 0.2) (layer "F.Cu") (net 6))
 (segment (start 218.33 61.835) (end 216.52 63.645) (width 0.2) (layer "F.Cu") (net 6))
 (segment (start 218.33 59.55) (end 218.33 61.835) (width 0.2) (layer "F.Cu") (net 6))
 (segment (start 210.07 50.0685) (end 212.3115 52.31) (width 0.2) (layer "F.Cu") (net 6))
 (via (at 218.43 59.45) (size 0.6) (drill 0.3) (layers "F.Cu" "B.Cu") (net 6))
 (via (at 213.11 52.31) (size 0.6) (drill 0.3) (layers "F.Cu" "B.Cu") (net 6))
 (segment (start 218.33 54.390057) (end 218.33 58.62) (width 0.2) (layer "B.Cu") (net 6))
 (segment (start 215.858943 51.919) (end 218.33 54.390057) (width 0.2) (layer "B.Cu") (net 6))
 (segment (start 218.33 58.62) (end 218.33 59.35) (width 0.2) (layer "B.Cu") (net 6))
 (segment (start 218.33 59.35) (end 218.43 59.45) (width 0.2) (layer "B.Cu") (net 6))
 (segment (start 213.501 51.919) (end 215.858943 51.919) (width 0.2) (layer "B.Cu") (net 6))
 (segment (start 213.11 52.31) (end 213.501 51.919) (width 0.2) (layer "B.Cu") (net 6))
 (segment (start 211.3785 52.6085) (end 211.81 53.04) (width 0.2) (layer "F.Cu") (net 5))
 (segment (start 210.07 52.6085) (end 211.3785 52.6085) (width 0.2) (layer "F.Cu") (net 5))
 (segment (start 212.43 62.095) (end 213.98 63.645) (width 0.2) (layer "F.Cu") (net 5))
 (segment (start 212.43 54.81) (end 212.43 62.095) (width 0.2) (layer "F.Cu") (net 5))
 (via (at 211.81 53.04) (size 0.6) (drill 0.3) (layers "F.Cu" "B.Cu") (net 5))
 (via (at 212.43 54.81) (size 0.6) (drill 0.3) (layers "F.Cu" "B.Cu") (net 5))
 (segment (start 212.43 53.66) (end 212.43 54.81) (width 0.2) (layer "B.Cu") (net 5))
 (segment (start 211.81 53.04) (end 212.43 53.66) (width 0.2) (layer "B.Cu") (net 5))
 (segment (start 254.97 45) (end 252.4185 42.4485) (width 0.2) (layer "F.Cu") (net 1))
 (segment (start 225.31 42.4485) (end 225.31 42.82) (width 0.2) (layer "F.Cu") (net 1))
 (segment (start 188.96 67.41) (end 205.135 67.41) (width 0.2) (layer "F.Cu") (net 1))
 (segment (start 205.135 67.41) (end 208.9 63.645) (width 0.2) (layer "F.Cu") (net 1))
 (segment (start 225.31 42.82) (end 215.61 52.52) (width 0.2) (layer "F.Cu") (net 1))
 (segment (start 252.4185 42.4485) (end 226.145 42.4485) (width 0.2) (layer "F.Cu") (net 1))
 (via (at 215.61 52.52) (size 0.6) (drill 0.3) (layers "F.Cu" "B.Cu") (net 1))
 (via (at 188.96 67.41) (size 0.6) (drill 0.3) (layers "F.Cu" "B.Cu") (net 1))
 (segment (start 185.67 64.12) (end 188.96 67.41) (width 0.2) (layer "B.Cu") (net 1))
 (segment (start 185.67 45.04) (end 185.67 64.12) (width 0.2) (layer "B.Cu") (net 1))
 (segment (start 254.91 81.23) (end 254.97 81.17) (width 0.2) (layer "B.Cu") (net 1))
 (segment (start 208.9 59.23) (end 208.9 63.645) (width 0.2) (layer "B.Cu") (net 1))
 (segment (start 254.97 81.17) (end 254.97 45) (width 0.2) (layer "B.Cu") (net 1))
 (segment (start 188.96 78.97) (end 185.63 82.3) (width 0.2) (layer "B.Cu") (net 1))
 (segment (start 254.91 82.28) (end 254.91 81.23) (width 0.2) (layer "B.Cu") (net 1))
 (segment (start 215.61 52.52) (end 208.9 59.23) (width 0.2) (layer "B.Cu") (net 1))
 (segment (start 188.96 67.41) (end 188.96 78.97) (width 0.2) (layer "B.Cu") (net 1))
 (segment (start 221.45 56.35) (end 222.6515 55.1485) (width 0.2) (layer "F.Cu") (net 2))
 (segment (start 222.6515 55.1485) (end 225.31 55.1485) (width 0.2) (layer "F.Cu") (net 2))
 (segment (start 179.32 47.58) (end 206.967874 47.58) (width 0.2) (layer "F.Cu") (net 2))
 (segment (start 206.967874 47.58) (end 207.979374 48.5915) (width 0.2) (layer "F.Cu") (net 2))
 (segment (start 213.7015 48.5915) (end 216.03 50.92) (width 0.2) (layer "F.Cu") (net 2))
 (segment (start 207.979374 48.5915) (end 213.7015 48.5915) (width 0.2) (layer "F.Cu") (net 2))
 (via (at 216.03 50.92) (size 0.6) (drill 0.3) (layers "F.Cu" "B.Cu") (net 2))
 (via (at 221.45 56.35) (size 0.6) (drill 0.3) (layers "F.Cu" "B.Cu") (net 2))
 (segment (start 216.03 50.92) (end 221.45 56.34) (width 0.2) (layer "B.Cu") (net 2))
 (segment (start 221.45 56.34) (end 221.45 56.35) (width 0.2) (layer "B.Cu") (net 2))
 (segment (start 179.28 84.84) (end 179.28 76.240057) (width 0.2) (layer "F.Cu") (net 8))
 (segment (start 179.28 76.240057) (end 201.848557 53.6715) (width 0.2) (layer "F.Cu") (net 8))
 (segment (start 201.848557 53.6715) (end 224.247 53.6715) (width 0.2) (layer "F.Cu") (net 8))
 (segment (start 224.247 53.6715) (end 225.31 52.6085) (width 0.2) (layer "F.Cu") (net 8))
 (segment (start 228.2265 52.15) (end 226.145 50.0685) (width 0.2) (layer "F.Cu") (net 3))
 (segment (start 229.35 52.15) (end 228.2265 52.15) (width 0.2) (layer "F.Cu") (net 3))
 (via (at 229.35 52.15) (size 0.6) (drill 0.3) (layers "F.Cu" "B.Cu") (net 3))
 (segment (start 233.96 47.54) (end 229.35 52.15) (width 0.2) (layer "B.Cu") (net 3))
 (segment (start 248.62 47.54) (end 233.96 47.54) (width 0.2) (layer "B.Cu") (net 3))
 (segment (start 248.56 69.9435) (end 226.145 47.5285) (width 0.2) (layer "F.Cu") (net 7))
 (segment (start 248.56 84.82) (end 248.56 69.9435) (width 0.2) (layer "F.Cu") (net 7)))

